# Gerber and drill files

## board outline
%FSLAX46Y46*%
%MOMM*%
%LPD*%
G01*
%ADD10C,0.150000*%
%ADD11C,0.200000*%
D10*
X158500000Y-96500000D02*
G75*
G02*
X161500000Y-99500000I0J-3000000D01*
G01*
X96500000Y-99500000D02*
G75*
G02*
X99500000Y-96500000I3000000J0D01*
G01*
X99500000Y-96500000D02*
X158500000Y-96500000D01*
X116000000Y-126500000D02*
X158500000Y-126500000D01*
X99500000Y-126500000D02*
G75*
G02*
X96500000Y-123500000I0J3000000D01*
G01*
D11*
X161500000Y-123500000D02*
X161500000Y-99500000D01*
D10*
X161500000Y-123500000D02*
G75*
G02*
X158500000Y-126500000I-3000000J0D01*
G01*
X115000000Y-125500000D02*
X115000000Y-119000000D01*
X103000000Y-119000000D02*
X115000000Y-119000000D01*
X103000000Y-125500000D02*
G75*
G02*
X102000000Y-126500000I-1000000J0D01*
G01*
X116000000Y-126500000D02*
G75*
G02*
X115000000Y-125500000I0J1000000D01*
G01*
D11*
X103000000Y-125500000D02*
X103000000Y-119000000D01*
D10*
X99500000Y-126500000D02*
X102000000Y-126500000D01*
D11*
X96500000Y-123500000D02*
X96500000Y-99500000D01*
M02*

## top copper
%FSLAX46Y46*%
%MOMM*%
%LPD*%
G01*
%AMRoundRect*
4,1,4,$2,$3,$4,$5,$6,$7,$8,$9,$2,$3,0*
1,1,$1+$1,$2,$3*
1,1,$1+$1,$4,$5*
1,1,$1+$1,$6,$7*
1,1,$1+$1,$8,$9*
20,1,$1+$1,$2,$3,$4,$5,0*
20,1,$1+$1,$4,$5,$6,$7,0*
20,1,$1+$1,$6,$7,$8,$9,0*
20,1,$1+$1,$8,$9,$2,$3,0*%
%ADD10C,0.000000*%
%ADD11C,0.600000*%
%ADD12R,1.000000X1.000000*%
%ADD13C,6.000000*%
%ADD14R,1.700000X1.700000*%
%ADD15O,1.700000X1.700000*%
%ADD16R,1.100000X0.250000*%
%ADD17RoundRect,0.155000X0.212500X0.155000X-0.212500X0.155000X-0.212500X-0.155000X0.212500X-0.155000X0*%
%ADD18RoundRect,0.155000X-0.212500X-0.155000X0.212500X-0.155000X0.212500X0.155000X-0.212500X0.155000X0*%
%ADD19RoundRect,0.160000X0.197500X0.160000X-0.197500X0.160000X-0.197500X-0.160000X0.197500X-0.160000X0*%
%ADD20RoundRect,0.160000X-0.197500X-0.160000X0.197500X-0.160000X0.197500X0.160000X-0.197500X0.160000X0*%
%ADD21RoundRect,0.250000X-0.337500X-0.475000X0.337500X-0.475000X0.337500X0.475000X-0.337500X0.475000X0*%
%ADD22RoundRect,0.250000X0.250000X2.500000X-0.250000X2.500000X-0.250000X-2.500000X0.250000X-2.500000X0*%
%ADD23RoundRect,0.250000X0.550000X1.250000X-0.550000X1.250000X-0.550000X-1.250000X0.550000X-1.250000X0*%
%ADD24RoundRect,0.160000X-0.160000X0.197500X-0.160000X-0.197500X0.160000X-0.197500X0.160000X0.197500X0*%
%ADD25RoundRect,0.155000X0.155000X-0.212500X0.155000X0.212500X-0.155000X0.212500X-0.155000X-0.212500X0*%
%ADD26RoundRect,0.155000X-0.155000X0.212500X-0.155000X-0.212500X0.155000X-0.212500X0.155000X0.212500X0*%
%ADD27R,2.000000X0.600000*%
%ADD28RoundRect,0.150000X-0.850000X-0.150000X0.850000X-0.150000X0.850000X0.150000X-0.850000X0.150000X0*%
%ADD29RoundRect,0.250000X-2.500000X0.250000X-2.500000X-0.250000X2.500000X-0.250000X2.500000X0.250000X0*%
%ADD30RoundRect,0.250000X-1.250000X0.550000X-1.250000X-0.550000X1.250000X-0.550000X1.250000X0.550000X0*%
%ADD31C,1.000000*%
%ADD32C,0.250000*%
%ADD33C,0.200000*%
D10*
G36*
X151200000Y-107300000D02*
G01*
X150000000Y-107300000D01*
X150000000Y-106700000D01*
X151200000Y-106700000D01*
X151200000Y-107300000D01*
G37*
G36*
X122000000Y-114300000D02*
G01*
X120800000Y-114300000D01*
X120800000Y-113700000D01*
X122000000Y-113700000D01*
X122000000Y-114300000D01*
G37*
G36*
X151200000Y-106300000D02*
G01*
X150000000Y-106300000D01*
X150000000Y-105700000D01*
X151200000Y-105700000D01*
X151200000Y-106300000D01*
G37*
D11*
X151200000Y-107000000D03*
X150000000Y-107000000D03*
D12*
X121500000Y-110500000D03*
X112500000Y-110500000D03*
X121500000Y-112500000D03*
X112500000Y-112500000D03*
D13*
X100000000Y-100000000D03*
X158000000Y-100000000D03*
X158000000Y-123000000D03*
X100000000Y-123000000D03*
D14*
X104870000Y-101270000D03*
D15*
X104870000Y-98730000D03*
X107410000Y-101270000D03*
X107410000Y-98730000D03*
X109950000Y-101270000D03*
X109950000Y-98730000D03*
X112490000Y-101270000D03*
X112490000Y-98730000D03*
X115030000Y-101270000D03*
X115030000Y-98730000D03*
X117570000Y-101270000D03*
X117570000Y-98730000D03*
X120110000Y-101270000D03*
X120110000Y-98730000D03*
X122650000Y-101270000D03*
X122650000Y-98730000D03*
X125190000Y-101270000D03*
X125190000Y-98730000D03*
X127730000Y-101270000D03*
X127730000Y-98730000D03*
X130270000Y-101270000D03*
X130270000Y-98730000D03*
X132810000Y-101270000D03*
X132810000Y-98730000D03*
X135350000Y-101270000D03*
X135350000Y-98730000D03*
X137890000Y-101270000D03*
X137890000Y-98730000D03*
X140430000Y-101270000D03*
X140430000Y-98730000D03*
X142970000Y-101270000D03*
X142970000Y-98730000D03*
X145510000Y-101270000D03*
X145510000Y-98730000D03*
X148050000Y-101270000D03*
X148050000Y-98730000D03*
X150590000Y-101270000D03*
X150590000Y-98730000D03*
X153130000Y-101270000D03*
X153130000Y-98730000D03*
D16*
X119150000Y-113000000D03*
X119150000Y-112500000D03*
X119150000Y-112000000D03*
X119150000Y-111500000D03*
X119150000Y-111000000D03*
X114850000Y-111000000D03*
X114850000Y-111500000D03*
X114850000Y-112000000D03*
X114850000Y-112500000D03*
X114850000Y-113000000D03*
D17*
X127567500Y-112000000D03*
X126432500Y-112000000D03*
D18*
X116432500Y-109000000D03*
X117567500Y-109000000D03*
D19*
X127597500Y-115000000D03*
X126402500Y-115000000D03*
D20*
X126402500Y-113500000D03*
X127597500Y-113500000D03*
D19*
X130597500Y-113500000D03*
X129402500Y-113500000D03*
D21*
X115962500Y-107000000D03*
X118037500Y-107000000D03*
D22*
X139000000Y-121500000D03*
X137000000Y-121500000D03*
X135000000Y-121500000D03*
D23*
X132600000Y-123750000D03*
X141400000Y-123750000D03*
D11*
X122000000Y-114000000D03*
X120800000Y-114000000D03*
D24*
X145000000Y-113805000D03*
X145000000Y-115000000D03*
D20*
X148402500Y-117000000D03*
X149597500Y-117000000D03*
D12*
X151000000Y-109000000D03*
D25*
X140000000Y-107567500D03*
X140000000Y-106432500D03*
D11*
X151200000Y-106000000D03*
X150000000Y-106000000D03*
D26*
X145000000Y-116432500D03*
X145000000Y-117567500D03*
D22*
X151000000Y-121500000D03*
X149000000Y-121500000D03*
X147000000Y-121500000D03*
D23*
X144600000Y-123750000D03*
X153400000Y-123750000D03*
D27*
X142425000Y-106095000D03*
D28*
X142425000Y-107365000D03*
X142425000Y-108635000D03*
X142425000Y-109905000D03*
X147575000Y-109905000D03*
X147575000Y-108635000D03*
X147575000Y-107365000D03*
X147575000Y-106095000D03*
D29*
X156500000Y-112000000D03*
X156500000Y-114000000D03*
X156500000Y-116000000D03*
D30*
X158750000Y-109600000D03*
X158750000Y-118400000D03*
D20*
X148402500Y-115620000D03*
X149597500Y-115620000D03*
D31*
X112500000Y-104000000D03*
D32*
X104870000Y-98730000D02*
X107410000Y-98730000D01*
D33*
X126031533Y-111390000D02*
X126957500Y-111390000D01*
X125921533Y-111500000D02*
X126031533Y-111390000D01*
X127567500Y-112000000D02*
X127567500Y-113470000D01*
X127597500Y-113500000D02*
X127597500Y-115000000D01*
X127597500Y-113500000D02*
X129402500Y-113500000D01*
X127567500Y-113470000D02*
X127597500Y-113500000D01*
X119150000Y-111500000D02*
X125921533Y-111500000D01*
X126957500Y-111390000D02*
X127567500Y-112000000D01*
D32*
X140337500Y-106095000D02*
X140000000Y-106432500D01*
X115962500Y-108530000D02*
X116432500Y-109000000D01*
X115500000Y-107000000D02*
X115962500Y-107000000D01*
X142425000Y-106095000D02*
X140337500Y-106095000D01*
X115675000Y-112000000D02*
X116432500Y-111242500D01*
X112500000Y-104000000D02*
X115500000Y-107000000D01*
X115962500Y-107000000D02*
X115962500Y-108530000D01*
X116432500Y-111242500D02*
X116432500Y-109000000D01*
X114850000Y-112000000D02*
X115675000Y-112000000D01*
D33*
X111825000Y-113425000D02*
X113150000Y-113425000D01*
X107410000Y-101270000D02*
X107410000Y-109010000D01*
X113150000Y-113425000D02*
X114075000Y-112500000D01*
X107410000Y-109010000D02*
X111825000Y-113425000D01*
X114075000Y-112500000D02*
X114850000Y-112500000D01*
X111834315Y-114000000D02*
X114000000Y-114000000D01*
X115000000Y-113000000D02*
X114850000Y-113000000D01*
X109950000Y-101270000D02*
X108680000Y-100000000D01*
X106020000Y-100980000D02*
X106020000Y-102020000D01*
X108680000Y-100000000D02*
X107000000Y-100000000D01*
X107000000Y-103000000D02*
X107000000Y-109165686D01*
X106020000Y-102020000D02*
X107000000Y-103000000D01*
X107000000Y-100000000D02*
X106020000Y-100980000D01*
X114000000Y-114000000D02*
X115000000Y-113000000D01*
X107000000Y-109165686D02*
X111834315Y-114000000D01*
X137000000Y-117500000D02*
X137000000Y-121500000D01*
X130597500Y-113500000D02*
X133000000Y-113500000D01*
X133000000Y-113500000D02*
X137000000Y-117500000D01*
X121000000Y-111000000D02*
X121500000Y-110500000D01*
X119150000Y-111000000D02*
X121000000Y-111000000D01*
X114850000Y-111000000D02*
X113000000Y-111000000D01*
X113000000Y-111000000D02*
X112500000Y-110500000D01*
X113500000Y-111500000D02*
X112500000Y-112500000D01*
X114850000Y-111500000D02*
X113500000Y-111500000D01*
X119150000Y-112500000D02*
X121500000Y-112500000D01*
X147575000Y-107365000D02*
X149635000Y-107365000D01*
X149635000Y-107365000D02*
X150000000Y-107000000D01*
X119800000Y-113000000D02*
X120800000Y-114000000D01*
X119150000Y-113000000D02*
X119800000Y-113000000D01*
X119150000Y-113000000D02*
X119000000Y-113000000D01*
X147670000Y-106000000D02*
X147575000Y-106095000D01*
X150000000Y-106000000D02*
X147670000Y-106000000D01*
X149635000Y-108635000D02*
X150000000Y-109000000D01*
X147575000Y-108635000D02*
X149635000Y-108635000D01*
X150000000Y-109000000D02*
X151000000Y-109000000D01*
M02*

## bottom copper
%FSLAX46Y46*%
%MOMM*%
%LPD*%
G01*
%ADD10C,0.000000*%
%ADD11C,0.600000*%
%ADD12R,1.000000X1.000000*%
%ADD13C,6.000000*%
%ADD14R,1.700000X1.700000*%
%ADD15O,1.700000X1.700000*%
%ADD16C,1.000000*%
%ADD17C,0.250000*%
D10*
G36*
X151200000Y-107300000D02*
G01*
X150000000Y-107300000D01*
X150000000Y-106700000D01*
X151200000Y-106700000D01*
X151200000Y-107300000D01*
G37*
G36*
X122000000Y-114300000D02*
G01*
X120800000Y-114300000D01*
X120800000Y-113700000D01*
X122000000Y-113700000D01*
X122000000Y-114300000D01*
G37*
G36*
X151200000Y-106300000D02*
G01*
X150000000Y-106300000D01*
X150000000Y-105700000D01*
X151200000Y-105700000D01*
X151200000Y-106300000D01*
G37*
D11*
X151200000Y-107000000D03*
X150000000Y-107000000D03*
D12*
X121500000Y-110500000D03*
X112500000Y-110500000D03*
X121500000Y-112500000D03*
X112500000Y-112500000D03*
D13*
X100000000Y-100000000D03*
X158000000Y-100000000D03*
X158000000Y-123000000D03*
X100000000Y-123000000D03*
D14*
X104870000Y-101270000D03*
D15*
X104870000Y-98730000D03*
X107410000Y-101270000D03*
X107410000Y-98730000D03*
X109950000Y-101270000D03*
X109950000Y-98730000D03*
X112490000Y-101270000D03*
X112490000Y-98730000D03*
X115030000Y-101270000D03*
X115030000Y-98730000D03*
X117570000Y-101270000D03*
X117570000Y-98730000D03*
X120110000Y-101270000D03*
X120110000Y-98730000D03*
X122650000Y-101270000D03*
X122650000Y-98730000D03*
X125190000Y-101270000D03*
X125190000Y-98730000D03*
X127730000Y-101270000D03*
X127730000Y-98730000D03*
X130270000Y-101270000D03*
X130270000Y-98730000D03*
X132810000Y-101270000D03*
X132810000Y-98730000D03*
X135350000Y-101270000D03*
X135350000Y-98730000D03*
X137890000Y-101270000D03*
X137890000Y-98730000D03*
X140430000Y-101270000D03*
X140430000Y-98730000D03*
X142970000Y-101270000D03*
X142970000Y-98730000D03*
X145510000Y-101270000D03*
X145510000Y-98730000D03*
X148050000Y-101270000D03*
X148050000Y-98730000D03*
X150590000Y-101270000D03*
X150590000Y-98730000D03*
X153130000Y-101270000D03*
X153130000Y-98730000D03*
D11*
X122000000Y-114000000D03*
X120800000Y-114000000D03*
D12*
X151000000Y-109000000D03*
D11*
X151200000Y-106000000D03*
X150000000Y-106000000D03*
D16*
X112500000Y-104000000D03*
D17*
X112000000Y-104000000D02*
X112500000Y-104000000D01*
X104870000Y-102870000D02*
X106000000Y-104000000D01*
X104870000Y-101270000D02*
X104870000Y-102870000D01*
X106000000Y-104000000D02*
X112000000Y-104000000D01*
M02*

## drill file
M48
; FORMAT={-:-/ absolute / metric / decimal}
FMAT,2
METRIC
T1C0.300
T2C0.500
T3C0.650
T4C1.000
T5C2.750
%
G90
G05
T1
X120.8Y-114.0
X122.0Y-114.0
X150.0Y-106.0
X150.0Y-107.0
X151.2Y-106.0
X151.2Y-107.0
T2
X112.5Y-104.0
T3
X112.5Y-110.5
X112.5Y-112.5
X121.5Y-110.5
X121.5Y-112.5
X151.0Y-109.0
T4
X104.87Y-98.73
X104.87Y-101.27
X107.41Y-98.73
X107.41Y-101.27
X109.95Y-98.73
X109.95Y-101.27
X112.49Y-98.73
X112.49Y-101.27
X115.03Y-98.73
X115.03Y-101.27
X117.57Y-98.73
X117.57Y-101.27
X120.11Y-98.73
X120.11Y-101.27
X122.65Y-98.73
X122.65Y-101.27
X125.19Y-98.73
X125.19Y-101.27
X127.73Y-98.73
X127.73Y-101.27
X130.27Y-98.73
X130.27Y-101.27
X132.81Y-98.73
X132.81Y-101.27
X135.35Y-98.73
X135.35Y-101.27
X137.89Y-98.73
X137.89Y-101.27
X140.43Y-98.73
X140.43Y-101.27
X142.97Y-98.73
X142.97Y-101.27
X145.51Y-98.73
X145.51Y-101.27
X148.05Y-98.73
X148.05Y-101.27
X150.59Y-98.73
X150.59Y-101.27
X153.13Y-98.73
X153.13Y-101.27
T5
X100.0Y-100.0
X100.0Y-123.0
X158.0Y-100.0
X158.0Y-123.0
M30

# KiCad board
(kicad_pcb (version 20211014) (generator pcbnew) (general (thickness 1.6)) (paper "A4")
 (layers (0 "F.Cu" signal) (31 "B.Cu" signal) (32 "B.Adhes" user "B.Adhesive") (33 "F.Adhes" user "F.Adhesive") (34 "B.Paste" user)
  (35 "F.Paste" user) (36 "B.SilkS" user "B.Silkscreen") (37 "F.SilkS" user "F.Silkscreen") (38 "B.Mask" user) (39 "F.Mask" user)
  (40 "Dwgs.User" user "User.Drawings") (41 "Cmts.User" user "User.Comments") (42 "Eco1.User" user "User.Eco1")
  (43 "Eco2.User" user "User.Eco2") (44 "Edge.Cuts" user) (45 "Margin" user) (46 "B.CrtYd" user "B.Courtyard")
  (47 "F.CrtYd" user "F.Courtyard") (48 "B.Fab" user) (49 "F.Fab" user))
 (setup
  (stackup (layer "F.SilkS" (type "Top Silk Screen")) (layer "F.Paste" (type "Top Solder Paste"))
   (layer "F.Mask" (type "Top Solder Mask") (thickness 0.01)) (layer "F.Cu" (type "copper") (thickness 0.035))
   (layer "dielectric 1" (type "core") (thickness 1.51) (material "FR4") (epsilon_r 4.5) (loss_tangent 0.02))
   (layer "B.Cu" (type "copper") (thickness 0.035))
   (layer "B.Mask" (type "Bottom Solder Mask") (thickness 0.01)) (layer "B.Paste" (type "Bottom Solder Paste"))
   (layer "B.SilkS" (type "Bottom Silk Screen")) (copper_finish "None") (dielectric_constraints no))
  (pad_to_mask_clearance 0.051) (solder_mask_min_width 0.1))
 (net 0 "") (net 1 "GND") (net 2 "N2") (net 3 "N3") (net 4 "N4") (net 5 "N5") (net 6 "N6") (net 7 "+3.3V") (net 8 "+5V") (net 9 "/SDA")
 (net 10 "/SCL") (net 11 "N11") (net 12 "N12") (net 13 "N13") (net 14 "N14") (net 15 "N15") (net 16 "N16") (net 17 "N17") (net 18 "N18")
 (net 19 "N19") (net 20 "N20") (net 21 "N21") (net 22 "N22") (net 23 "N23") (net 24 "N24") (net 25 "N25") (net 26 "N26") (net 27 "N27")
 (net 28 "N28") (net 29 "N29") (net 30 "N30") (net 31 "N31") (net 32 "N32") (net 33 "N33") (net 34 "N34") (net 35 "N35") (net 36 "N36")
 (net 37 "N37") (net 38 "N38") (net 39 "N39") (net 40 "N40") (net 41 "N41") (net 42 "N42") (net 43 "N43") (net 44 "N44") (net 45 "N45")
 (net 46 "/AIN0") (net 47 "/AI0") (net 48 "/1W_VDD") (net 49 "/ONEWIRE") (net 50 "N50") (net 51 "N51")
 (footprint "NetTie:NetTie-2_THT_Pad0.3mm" (layer "F.Cu") (at 151.2 107 180)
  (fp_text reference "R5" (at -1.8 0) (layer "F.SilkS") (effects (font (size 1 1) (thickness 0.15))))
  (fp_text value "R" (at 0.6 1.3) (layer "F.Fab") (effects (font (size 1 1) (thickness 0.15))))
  (fp_poly (pts (xy 0 -0.3) (xy 1.2 -0.3) (xy 1.2 0.3) (xy 0 0.3)) (layer "F.Cu") (width 0) (fill solid))
  (fp_poly (pts (xy 0 -0.3) (xy 1.2 -0.3) (xy 1.2 0.3) (xy 0 0.3)) (layer "B.Cu") (width 0) (fill solid))
  (pad "1" thru_hole circle (at 0 0 180) (size 0.6 0.6) (drill 0.3) (layers *.Cu) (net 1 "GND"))
  (pad "2" thru_hole circle (at 1.2 0 180) (size 0.6 0.6) (drill 0.3) (layers *.Cu) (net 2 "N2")))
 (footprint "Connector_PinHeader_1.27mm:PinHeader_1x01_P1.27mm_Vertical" (layer "F.Cu") (at 121.5 110.5 -90)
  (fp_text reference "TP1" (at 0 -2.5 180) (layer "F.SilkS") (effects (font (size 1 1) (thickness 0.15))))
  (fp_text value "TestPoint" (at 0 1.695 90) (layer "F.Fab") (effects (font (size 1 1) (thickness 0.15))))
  (pad "1" thru_hole rect (at 0 0 270) (size 1 1) (drill 0.65) (layers *.Cu *.Mask) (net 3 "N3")))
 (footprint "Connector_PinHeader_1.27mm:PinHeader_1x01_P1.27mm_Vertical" (layer "F.Cu") (at 112.5 110.5 90)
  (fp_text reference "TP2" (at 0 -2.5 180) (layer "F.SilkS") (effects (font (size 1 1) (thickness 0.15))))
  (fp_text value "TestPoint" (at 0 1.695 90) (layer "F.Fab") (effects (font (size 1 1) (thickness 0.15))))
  (pad "1" thru_hole rect (at 0 0 90) (size 1 1) (drill 0.65) (layers *.Cu *.Mask) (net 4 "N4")))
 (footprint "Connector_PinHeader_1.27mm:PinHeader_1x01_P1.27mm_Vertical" (layer "F.Cu") (at 121.5 112.5 -90)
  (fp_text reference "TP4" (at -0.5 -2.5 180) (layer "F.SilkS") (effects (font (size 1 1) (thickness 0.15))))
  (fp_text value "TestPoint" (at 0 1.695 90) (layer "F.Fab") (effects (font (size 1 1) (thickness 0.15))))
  (pad "1" thru_hole rect (at 0 0 270) (size 1 1) (drill 0.65) (layers *.Cu *.Mask) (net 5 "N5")))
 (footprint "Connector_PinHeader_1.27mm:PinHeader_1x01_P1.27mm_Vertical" (layer "F.Cu") (at 112.5 112.5 90)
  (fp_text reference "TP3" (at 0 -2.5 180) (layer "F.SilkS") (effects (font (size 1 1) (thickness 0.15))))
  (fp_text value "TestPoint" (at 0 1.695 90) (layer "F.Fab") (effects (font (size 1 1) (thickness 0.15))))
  (pad "1" thru_hole rect (at 0 0 90) (size 1 1) (drill 0.65) (layers *.Cu *.Mask) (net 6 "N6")))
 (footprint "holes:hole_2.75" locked (layer "F.Cu") (at 100 100)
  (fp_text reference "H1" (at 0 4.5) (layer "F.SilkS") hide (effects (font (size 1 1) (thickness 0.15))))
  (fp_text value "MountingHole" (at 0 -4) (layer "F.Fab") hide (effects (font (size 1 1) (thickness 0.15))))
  (pad "" np_thru_hole circle locked (at 0 0) (size 6 6) (drill 2.75) (layers *.Cu *.Mask)))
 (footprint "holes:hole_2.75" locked (layer "F.Cu") (at 158 100)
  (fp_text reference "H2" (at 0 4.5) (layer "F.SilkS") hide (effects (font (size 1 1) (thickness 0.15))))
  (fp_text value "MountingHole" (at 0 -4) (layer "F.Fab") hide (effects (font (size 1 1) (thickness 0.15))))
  (pad "" np_thru_hole circle locked (at 0 0) (size 6 6) (drill 2.75) (layers *.Cu *.Mask)))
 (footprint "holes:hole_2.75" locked (layer "F.Cu") (at 158 123)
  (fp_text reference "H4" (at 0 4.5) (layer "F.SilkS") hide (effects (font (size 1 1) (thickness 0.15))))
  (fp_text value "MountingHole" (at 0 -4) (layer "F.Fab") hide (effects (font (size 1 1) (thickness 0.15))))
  (pad "" np_thru_hole circle locked (at 0 0) (size 6 6) (drill 2.75) (layers *.Cu *.Mask)))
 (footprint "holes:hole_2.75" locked (layer "F.Cu") (at 100 123)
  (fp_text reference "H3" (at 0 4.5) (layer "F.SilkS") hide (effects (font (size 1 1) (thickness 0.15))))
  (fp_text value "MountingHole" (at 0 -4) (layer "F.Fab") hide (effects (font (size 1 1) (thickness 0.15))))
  (pad "" np_thru_hole circle locked (at 0 0) (size 6 6) (drill 2.75) (layers *.Cu *.Mask)))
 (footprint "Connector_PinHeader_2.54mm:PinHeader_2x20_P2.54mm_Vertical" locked (layer "F.Cu") (at 104.87 101.27 90)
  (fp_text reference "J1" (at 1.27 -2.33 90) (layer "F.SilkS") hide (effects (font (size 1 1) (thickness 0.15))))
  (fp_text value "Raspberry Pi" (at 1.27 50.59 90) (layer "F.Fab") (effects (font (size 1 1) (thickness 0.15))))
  (pad "1" thru_hole rect locked (at 0 0 90) (size 1.7 1.7) (drill 1) (layers *.Cu *.Mask) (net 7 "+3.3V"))
  (pad "2" thru_hole oval locked (at 2.54 0 90) (size 1.7 1.7) (drill 1) (layers *.Cu *.Mask) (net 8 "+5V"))
  (pad "3" thru_hole oval locked (at 0 2.54 90) (size 1.7 1.7) (drill 1) (layers *.Cu *.Mask) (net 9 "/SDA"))
  (pad "4" thru_hole oval locked (at 2.54 2.54 90) (size 1.7 1.7) (drill 1) (layers *.Cu *.Mask) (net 8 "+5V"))
  (pad "5" thru_hole oval locked (at 0 5.08 90) (size 1.7 1.7) (drill 1) (layers *.Cu *.Mask) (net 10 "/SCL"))
  (pad "6" thru_hole oval locked (at 2.54 5.08 90) (size 1.7 1.7) (drill 1) (layers *.Cu *.Mask) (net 1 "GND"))
  (pad "7" thru_hole oval locked (at 0 7.62 90) (size 1.7 1.7) (drill 1) (layers *.Cu *.Mask) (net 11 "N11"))
  (pad "8" thru_hole oval locked (at 2.54 7.62 90) (size 1.7 1.7) (drill 1) (layers *.Cu *.Mask) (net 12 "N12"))
  (pad "9" thru_hole oval locked (at 0 10.16 90) (size 1.7 1.7) (drill 1) (layers *.Cu *.Mask) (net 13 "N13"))
  (pad "10" thru_hole oval locked (at 2.54 10.16 90) (size 1.7 1.7) (drill 1) (layers *.Cu *.Mask) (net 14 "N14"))
  (pad "11" thru_hole oval locked (at 0 12.7 90) (size 1.7 1.7) (drill 1) (layers *.Cu *.Mask) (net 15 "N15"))
  (pad "12" thru_hole oval locked (at 2.54 12.7 90) (size 1.7 1.7) (drill 1) (layers *.Cu *.Mask) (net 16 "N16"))
  (pad "13" thru_hole oval locked (at 0 15.24 90) (size 1.7 1.7) (drill 1) (layers *.Cu *.Mask) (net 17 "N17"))
  (pad "14" thru_hole oval locked (at 2.54 15.24 90) (size 1.7 1.7) (drill 1) (layers *.Cu *.Mask) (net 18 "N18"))
  (pad "15" thru_hole oval locked (at 0 17.78 90) (size 1.7 1.7) (drill 1) (layers *.Cu *.Mask) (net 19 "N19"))
  (pad "16" thru_hole oval locked (at 2.54 17.78 90) (size 1.7 1.7) (drill 1) (layers *.Cu *.Mask) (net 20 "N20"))
  (pad "17" thru_hole oval locked (at 0 20.32 90) (size 1.7 1.7) (drill 1) (layers *.Cu *.Mask) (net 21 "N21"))
  (pad "18" thru_hole oval locked (at 2.54 20.32 90) (size 1.7 1.7) (drill 1) (layers *.Cu *.Mask) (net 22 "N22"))
  (pad "19" thru_hole oval locked (at 0 22.86 90) (size 1.7 1.7) (drill 1) (layers *.Cu *.Mask) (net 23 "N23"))
  (pad "20" thru_hole oval locked (at 2.54 22.86 90) (size 1.7 1.7) (drill 1) (layers *.Cu *.Mask) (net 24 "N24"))
  (pad "21" thru_hole oval locked (at 0 25.4 90) (size 1.7 1.7) (drill 1) (layers *.Cu *.Mask) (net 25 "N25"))
  (pad "22" thru_hole oval locked (at 2.54 25.4 90) (size 1.7 1.7) (drill 1) (layers *.Cu *.Mask) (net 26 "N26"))
  (pad "23" thru_hole oval locked (at 0 27.94 90) (size 1.7 1.7) (drill 1) (layers *.Cu *.Mask) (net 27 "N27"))
  (pad "24" thru_hole oval locked (at 2.54 27.94 90) (size 1.7 1.7) (drill 1) (layers *.Cu *.Mask) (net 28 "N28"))
  (pad "25" thru_hole oval locked (at 0 30.48 90) (size 1.7 1.7) (drill 1) (layers *.Cu *.Mask) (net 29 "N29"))
  (pad "26" thru_hole oval locked (at 2.54 30.48 90) (size 1.7 1.7) (drill 1) (layers *.Cu *.Mask) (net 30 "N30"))
  (pad "27" thru_hole oval locked (at 0 33.02 90) (size 1.7 1.7) (drill 1) (layers *.Cu *.Mask) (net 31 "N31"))
  (pad "28" thru_hole oval locked (at 2.54 33.02 90) (size 1.7 1.7) (drill 1) (layers *.Cu *.Mask) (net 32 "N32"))
  (pad "29" thru_hole oval locked (at 0 35.56 90) (size 1.7 1.7) (drill 1) (layers *.Cu *.Mask) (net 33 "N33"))
  (pad "30" thru_hole oval locked (at 2.54 35.56 90) (size 1.7 1.7) (drill 1) (layers *.Cu *.Mask) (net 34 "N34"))
  (pad "31" thru_hole oval locked (at 0 38.1 90) (size 1.7 1.7) (drill 1) (layers *.Cu *.Mask) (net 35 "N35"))
  (pad "32" thru_hole oval locked (at 2.54 38.1 90) (size 1.7 1.7) (drill 1) (layers *.Cu *.Mask) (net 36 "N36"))
  (pad "33" thru_hole oval locked (at 0 40.64 90) (size 1.7 1.7) (drill 1) (layers *.Cu *.Mask) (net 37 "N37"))
  (pad "34" thru_hole oval locked (at 2.54 40.64 90) (size 1.7 1.7) (drill 1) (layers *.Cu *.Mask) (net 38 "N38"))
  (pad "35" thru_hole oval locked (at 0 43.18 90) (size 1.7 1.7) (drill 1) (layers *.Cu *.Mask) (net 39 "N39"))
  (pad "36" thru_hole oval locked (at 2.54 43.18 90) (size 1.7 1.7) (drill 1) (layers *.Cu *.Mask) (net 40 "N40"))
  (pad "37" thru_hole oval locked (at 0 45.72 90) (size 1.7 1.7) (drill 1) (layers *.Cu *.Mask) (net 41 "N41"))
  (pad "38" thru_hole oval locked (at 2.54 45.72 90) (size 1.7 1.7) (drill 1) (layers *.Cu *.Mask) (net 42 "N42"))
  (pad "39" thru_hole oval locked (at 0 48.26 90) (size 1.7 1.7) (drill 1) (layers *.Cu *.Mask) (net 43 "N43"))
  (pad "40" thru_hole oval locked (at 2.54 48.26 90) (size 1.7 1.7) (drill 1) (layers *.Cu *.Mask) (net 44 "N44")))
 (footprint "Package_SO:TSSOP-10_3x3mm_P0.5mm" (layer "F.Cu") (at 117 112 180)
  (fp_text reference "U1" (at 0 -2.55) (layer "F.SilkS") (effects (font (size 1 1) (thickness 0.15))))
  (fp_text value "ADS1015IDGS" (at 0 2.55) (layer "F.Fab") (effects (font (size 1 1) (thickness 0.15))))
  (pad "1" smd rect (at -2.15 -1 180) (size 1.1 0.25) (layers "F.Cu" "F.Paste" "F.Mask") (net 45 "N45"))
  (pad "2" smd rect (at -2.15 -0.5 180) (size 1.1 0.25) (layers "F.Cu" "F.Paste" "F.Mask") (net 5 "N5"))
  (pad "3" smd rect (at -2.15 0 180) (size 1.1 0.25) (layers "F.Cu" "F.Paste" "F.Mask") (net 1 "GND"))
  (pad "4" smd rect (at -2.15 0.5 180) (size 1.1 0.25) (layers "F.Cu" "F.Paste" "F.Mask") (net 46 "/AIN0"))
  (pad "5" smd rect (at -2.15 1 180) (size 1.1 0.25) (layers "F.Cu" "F.Paste" "F.Mask") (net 3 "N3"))
  (pad "6" smd rect (at 2.15 1 180) (size 1.1 0.25) (layers "F.Cu" "F.Paste" "F.Mask") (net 4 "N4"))
  (pad "7" smd rect (at 2.15 0.5 180) (size 1.1 0.25) (layers "F.Cu" "F.Paste" "F.Mask") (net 6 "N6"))
  (pad "8" smd rect (at 2.15 0 180) (size 1.1 0.25) (layers "F.Cu" "F.Paste" "F.Mask") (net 7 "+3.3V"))
  (pad "9" smd rect (at 2.15 -0.5 180) (size 1.1 0.25) (layers "F.Cu" "F.Paste" "F.Mask") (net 9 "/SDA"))
  (pad "10" smd rect (at 2.15 -1 180) (size 1.1 0.25) (layers "F.Cu" "F.Paste" "F.Mask") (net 10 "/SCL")))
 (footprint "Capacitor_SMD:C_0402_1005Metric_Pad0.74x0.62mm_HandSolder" (layer "F.Cu") (at 127 112 180)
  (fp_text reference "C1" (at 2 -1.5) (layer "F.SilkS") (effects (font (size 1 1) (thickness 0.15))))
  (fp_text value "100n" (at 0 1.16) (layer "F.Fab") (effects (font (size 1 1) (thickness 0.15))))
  (pad "1" smd roundrect (at -0.5675 0 180) (size 0.735 0.62) (layers "F.Cu" "F.Paste" "F.Mask") (roundrect_rratio 0.25) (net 46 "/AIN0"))
  (pad "2" smd roundrect (at 0.5675 0 180) (size 0.735 0.62) (layers "F.Cu" "F.Paste" "F.Mask") (roundrect_rratio 0.25) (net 1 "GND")))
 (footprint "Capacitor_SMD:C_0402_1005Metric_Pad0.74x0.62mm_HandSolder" (layer "F.Cu") (at 117 109)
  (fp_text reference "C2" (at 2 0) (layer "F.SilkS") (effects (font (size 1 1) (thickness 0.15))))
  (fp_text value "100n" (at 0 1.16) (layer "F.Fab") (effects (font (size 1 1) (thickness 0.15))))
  (pad "1" smd roundrect (at -0.5675 0) (size 0.735 0.62) (layers "F.Cu" "F.Paste" "F.Mask") (roundrect_rratio 0.25) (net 7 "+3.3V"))
  (pad "2" smd roundrect (at 0.5675 0) (size 0.735 0.62) (layers "F.Cu" "F.Paste" "F.Mask") (roundrect_rratio 0.25) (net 1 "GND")))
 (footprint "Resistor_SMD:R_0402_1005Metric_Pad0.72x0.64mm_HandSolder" (layer "F.Cu") (at 127 115 180)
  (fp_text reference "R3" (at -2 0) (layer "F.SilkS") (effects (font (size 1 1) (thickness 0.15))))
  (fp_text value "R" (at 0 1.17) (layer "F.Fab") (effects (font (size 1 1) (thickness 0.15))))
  (pad "1" smd roundrect (at -0.5975 0 180) (size 0.715 0.64) (layers "F.Cu" "F.Paste" "F.Mask") (roundrect_rratio 0.25) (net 46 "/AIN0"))
  (pad "2" smd roundrect (at 0.5975 0 180) (size 0.715 0.64) (layers "F.Cu" "F.Paste" "F.Mask") (roundrect_rratio 0.25) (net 7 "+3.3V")))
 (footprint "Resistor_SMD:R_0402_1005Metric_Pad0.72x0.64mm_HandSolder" (layer "F.Cu") (at 127 113.5)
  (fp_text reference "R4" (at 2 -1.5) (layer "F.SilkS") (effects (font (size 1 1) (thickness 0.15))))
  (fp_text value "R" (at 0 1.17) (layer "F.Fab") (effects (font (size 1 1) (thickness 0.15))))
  (pad "1" smd roundrect (at -0.5975 0) (size 0.715 0.64) (layers "F.Cu" "F.Paste" "F.Mask") (roundrect_rratio 0.25) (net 1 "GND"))
  (pad "2" smd roundrect (at 0.5975 0) (size 0.715 0.64) (layers "F.Cu" "F.Paste" "F.Mask") (roundrect_rratio 0.25) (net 46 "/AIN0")))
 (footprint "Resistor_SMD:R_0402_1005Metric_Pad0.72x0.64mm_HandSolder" (layer "F.Cu") (at 130 113.5 180)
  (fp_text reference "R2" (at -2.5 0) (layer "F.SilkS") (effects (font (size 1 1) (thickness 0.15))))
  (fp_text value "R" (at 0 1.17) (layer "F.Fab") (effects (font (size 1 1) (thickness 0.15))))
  (pad "1" smd roundrect (at -0.5975 0 180) (size 0.715 0.64) (layers "F.Cu" "F.Paste" "F.Mask") (roundrect_rratio 0.25) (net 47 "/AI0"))
  (pad "2" smd roundrect (at 0.5975 0 180) (size 0.715 0.64) (layers "F.Cu" "F.Paste" "F.Mask") (roundrect_rratio 0.25) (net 46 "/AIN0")))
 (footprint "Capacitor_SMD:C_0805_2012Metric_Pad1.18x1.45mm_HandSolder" (layer "F.Cu") (at 117 107)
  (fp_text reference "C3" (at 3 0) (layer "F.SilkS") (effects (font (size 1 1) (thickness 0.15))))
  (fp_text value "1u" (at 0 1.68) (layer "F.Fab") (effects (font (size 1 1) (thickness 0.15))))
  (pad "1" smd roundrect (at -1.0375 0) (size 1.175 1.45) (layers "F.Cu" "F.Paste" "F.Mask") (roundrect_rratio 0.212766) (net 7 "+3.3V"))
  (pad "2" smd roundrect (at 1.0375 0) (size 1.175 1.45) (layers "F.Cu" "F.Paste" "F.Mask") (roundrect_rratio 0.212766) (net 1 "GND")))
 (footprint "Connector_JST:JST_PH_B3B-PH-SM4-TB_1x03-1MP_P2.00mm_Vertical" (layer "F.Cu") (at 137 122 180)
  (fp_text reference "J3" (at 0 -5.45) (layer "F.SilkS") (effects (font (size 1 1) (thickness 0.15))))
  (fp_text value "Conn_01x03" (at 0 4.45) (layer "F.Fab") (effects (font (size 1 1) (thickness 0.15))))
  (pad "1" smd roundrect (at -2 0.5 180) (size 1 5.5) (layers "F.Cu" "F.Paste" "F.Mask") (roundrect_rratio 0.25) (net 1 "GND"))
  (pad "2" smd roundrect (at 0 0.5 180) (size 1 5.5) (layers "F.Cu" "F.Paste" "F.Mask") (roundrect_rratio 0.25) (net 47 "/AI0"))
  (pad "3" smd roundrect (at 2 0.5 180) (size 1 5.5) (layers "F.Cu" "F.Paste" "F.Mask") (roundrect_rratio 0.25) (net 7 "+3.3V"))
  (pad "MP" smd roundrect (at 4.4 -1.75 180) (size 1.6 3) (layers "F.Cu" "F.Paste" "F.Mask") (roundrect_rratio 0.15625))
  (pad "MP" smd roundrect (at -4.4 -1.75 180) (size 1.6 3) (layers "F.Cu" "F.Paste" "F.Mask") (roundrect_rratio 0.15625)))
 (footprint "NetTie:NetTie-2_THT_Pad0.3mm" (layer "F.Cu") (at 122 114 180)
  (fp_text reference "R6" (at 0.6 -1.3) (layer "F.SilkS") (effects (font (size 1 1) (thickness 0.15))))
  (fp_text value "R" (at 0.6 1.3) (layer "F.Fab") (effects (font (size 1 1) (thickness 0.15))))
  (fp_poly (pts (xy 0 -0.3) (xy 1.2 -0.3) (xy 1.2 0.3) (xy 0 0.3)) (layer "F.Cu") (width 0) (fill solid))
  (fp_poly (pts (xy 0 -0.3) (xy 1.2 -0.3) (xy 1.2 0.3) (xy 0 0.3)) (layer "B.Cu") (width 0) (fill solid))
  (pad "1" thru_hole circle (at 0 0 180) (size 0.6 0.6) (drill 0.3) (layers *.Cu) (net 1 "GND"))
  (pad "2" thru_hole circle (at 1.2 0 180) (size 0.6 0.6) (drill 0.3) (layers *.Cu) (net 45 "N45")))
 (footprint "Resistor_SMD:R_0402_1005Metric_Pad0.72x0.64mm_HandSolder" (layer "F.Cu") (at 145 114.4025 -90)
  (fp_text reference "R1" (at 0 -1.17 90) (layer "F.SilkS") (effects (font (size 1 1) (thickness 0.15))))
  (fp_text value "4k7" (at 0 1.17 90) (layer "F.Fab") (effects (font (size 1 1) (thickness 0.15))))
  (pad "1" smd roundrect (at -0.5975 0 270) (size 0.715 0.64) (layers "F.Cu" "F.Paste" "F.Mask") (roundrect_rratio 0.25) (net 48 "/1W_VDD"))
  (pad "2" smd roundrect (at 0.5975 0 270) (size 0.715 0.64) (layers "F.Cu" "F.Paste" "F.Mask") (roundrect_rratio 0.25) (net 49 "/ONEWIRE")))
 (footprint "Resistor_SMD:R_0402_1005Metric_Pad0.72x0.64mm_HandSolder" (layer "F.Cu") (at 149 117)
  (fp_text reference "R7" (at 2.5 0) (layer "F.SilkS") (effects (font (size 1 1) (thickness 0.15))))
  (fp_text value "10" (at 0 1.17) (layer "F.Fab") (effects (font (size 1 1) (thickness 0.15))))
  (pad "1" smd roundrect (at -0.5975 0) (size 0.715 0.64) (layers "F.Cu" "F.Paste" "F.Mask") (roundrect_rratio 0.25) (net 11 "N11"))
  (pad "2" smd roundrect (at 0.5975 0) (size 0.715 0.64) (layers "F.Cu" "F.Paste" "F.Mask") (roundrect_rratio 0.25) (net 49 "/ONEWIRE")))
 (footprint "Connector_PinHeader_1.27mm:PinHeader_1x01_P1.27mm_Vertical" (layer "F.Cu") (at 151 109)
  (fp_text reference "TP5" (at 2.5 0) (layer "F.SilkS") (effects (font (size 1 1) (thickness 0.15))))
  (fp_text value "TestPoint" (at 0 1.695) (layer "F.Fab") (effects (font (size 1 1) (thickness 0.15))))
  (pad "1" thru_hole rect (at 0 0) (size 1 1) (drill 0.65) (layers *.Cu *.Mask) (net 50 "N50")))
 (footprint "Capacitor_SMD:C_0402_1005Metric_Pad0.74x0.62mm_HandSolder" (layer "F.Cu") (at 140 107 90)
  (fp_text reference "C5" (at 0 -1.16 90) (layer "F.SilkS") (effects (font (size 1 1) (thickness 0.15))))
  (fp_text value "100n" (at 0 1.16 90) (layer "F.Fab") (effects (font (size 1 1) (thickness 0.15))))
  (pad "1" smd roundrect (at -0.5675 0 90) (size 0.735 0.62) (layers "F.Cu" "F.Paste" "F.Mask") (roundrect_rratio 0.25) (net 1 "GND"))
  (pad "2" smd roundrect (at 0.5675 0 90) (size 0.735 0.62) (layers "F.Cu" "F.Paste" "F.Mask") (roundrect_rratio 0.25) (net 7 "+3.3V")))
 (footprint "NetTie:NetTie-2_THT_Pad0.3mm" (layer "F.Cu") (at 151.2 106 180)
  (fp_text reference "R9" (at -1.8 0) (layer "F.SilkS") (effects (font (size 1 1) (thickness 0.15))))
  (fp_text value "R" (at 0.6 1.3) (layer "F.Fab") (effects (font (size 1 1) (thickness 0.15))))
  (fp_poly (pts (xy 0 -0.3) (xy 1.2 -0.3) (xy 1.2 0.3) (xy 0 0.3)) (layer "F.Cu") (width 0) (fill solid))
  (fp_poly (pts (xy 0 -0.3) (xy 1.2 -0.3) (xy 1.2 0.3) (xy 0 0.3)) (layer "B.Cu") (width 0) (fill solid))
  (pad "1" thru_hole circle (at 0 0 180) (size 0.6 0.6) (drill 0.3) (layers *.Cu) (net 1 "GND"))
  (pad "2" thru_hole circle (at 1.2 0 180) (size 0.6 0.6) (drill 0.3) (layers *.Cu) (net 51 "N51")))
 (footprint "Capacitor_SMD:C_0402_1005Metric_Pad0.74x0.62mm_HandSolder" (layer "F.Cu") (at 145 117 -90)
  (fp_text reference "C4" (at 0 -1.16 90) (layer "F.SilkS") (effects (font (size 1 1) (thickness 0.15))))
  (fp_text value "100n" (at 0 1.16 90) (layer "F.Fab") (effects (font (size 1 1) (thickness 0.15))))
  (pad "1" smd roundrect (at -0.5675 0 270) (size 0.735 0.62) (layers "F.Cu" "F.Paste" "F.Mask") (roundrect_rratio 0.25) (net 1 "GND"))
  (pad "2" smd roundrect (at 0.5675 0 270) (size 0.735 0.62) (layers "F.Cu" "F.Paste" "F.Mask") (roundrect_rratio 0.25) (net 48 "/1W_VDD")))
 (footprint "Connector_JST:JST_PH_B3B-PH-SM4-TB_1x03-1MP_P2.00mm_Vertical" (layer "F.Cu") (at 149 122 180)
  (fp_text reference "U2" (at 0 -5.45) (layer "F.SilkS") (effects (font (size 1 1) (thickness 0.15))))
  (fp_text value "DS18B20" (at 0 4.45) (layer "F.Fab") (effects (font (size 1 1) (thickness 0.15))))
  (pad "1" smd roundrect (at -2 0.5 180) (size 1 5.5) (layers "F.Cu" "F.Paste" "F.Mask") (roundrect_rratio 0.25) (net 1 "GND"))
  (pad "2" smd roundrect (at 0 0.5 180) (size 1 5.5) (layers "F.Cu" "F.Paste" "F.Mask") (roundrect_rratio 0.25) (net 49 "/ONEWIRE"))
  (pad "3" smd roundrect (at 2 0.5 180) (size 1 5.5) (layers "F.Cu" "F.Paste" "F.Mask") (roundrect_rratio 0.25) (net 48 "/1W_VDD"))
  (pad "MP" smd roundrect (at 4.4 -1.75 180) (size 1.6 3) (layers "F.Cu" "F.Paste" "F.Mask") (roundrect_rratio 0.15625))
  (pad "MP" smd roundrect (at -4.4 -1.75 180) (size 1.6 3) (layers "F.Cu" "F.Paste" "F.Mask") (roundrect_rratio 0.15625)))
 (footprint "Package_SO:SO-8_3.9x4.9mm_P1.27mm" (layer "F.Cu") (at 145 108)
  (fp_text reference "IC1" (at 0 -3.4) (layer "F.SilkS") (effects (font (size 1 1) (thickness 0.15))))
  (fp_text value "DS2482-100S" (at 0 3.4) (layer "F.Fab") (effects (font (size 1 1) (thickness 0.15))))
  (pad "1" smd rect (at -2.575 -1.905) (size 2 0.6) (layers "F.Cu" "F.Paste" "F.Mask") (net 7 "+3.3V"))
  (pad "2" smd roundrect (at -2.575 -0.635) (size 2 0.6) (layers "F.Cu" "F.Paste" "F.Mask") (roundrect_rratio 0.25) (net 49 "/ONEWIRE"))
  (pad "3" smd roundrect (at -2.575 0.635) (size 2 0.6) (layers "F.Cu" "F.Paste" "F.Mask") (roundrect_rratio 0.25) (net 1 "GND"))
  (pad "4" smd roundrect (at -2.575 1.905) (size 2 0.6) (layers "F.Cu" "F.Paste" "F.Mask") (roundrect_rratio 0.25) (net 10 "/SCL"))
  (pad "5" smd roundrect (at 2.575 1.905) (size 2 0.6) (layers "F.Cu" "F.Paste" "F.Mask") (roundrect_rratio 0.25) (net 9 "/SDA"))
  (pad "6" smd roundrect (at 2.575 0.635) (size 2 0.6) (layers "F.Cu" "F.Paste" "F.Mask") (roundrect_rratio 0.25) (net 50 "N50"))
  (pad "7" smd roundrect (at 2.575 -0.635) (size 2 0.6) (layers "F.Cu" "F.Paste" "F.Mask") (roundrect_rratio 0.25) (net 2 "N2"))
  (pad "8" smd roundrect (at 2.575 -1.905) (size 2 0.6) (layers "F.Cu" "F.Paste" "F.Mask") (roundrect_rratio 0.25) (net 51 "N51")))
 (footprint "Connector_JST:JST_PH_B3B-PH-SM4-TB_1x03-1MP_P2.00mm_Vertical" (layer "F.Cu") (at 157 114 -90)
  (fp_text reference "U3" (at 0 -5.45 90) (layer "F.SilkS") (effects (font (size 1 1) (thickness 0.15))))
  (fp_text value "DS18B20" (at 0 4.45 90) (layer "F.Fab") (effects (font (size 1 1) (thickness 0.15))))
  (pad "1" smd roundrect (at -2 0.5 270) (size 1 5.5) (layers "F.Cu" "F.Paste" "F.Mask") (roundrect_rratio 0.25) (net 1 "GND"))
  (pad "2" smd roundrect (at 0 0.5 270) (size 1 5.5) (layers "F.Cu" "F.Paste" "F.Mask") (roundrect_rratio 0.25) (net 49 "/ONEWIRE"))
  (pad "3" smd roundrect (at 2 0.5 270) (size 1 5.5) (layers "F.Cu" "F.Paste" "F.Mask") (roundrect_rratio 0.25) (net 48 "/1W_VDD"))
  (pad "MP" smd roundrect (at -4.4 -1.75 270) (size 1.6 3) (layers "F.Cu" "F.Paste" "F.Mask") (roundrect_rratio 0.15625))
  (pad "MP" smd roundrect (at 4.4 -1.75 270) (size 1.6 3) (layers "F.Cu" "F.Paste" "F.Mask") (roundrect_rratio 0.15625)))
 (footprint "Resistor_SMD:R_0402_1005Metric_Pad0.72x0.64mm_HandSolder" (layer "F.Cu") (at 149 115.62)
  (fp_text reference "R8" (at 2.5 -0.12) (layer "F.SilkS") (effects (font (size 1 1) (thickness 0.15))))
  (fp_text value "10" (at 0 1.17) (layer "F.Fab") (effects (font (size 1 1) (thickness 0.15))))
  (pad "1" smd roundrect (at -0.5975 0) (size 0.715 0.64) (layers "F.Cu" "F.Paste" "F.Mask") (roundrect_rratio 0.25) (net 7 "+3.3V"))
  (pad "2" smd roundrect (at 0.5975 0) (size 0.715 0.64) (layers "F.Cu" "F.Paste" "F.Mask") (roundrect_rratio 0.25) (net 48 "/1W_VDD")))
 (gr_arc (start 158.5 96.5) (mid 160.62132 97.37868) (end 161.5 99.5) (layer "Edge.Cuts") (width 0.15))
 (gr_arc (start 96.5 99.5) (mid 97.37868 97.37868) (end 99.5 96.5) (layer "Edge.Cuts") (width 0.15))
 (gr_line (start 99.5 96.5) (end 158.5 96.5) (layer "Edge.Cuts") (width 0.15))
 (gr_line (start 116 126.5) (end 158.5 126.5) (layer "Edge.Cuts") (width 0.15))
 (gr_arc (start 99.5 126.5) (mid 97.37868 125.62132) (end 96.5 123.5) (layer "Edge.Cuts") (width 0.15))
 (gr_line (start 161.5 123.5) (end 161.5 99.5) (layer "Edge.Cuts") (width 0.2))
 (gr_arc (start 161.5 123.5) (mid 160.62132 125.62132) (end 158.5 126.5) (layer "Edge.Cuts") (width 0.15))
 (gr_line (start 115 125.5) (end 115 119) (layer "Edge.Cuts") (width 0.15))
 (gr_line (start 103 119) (end 115 119) (layer "Edge.Cuts") (width 0.15))
 (gr_arc (start 103 125.5) (mid 102.707107 126.207107) (end 102 126.5) (layer "Edge.Cuts") (width 0.15))
 (gr_arc (start 116 126.5) (mid 115.292893 126.207107) (end 115 125.5) (layer "Edge.Cuts") (width 0.15))
 (gr_line (start 103 125.5) (end 103 119) (layer "Edge.Cuts") (width 0.2))
 (gr_line (start 99.5 126.5) (end 102 126.5) (layer "Edge.Cuts") (width 0.15))
 (gr_line (start 96.5 123.5) (end 96.5 99.5) (layer "Edge.Cuts") (width 0.2))
 (segment (start 104.87 98.73) (end 107.41 98.73) (width 0.25) (layer "F.Cu") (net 8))
 (segment (start 126.031533 111.39) (end 126.9575 111.39) (width 0.2) (layer "F.Cu") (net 46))
 (segment (start 125.921533 111.5) (end 126.031533 111.39) (width 0.2) (layer "F.Cu") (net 46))
 (segment (start 127.5675 112) (end 127.5675 113.47) (width 0.2) (layer "F.Cu") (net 46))
 (segment (start 127.5975 113.5) (end 127.5975 115) (width 0.2) (layer "F.Cu") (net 46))
 (segment (start 127.5975 113.5) (end 129.4025 113.5) (width 0.2) (layer "F.Cu") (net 46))
 (segment (start 127.5675 113.47) (end 127.5975 113.5) (width 0.2) (layer "F.Cu") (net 46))
 (segment (start 119.15 111.5) (end 125.921533 111.5) (width 0.2) (layer "F.Cu") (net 46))
 (segment (start 126.9575 111.39) (end 127.5675 112) (width 0.2) (layer "F.Cu") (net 46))
 (segment (start 140.3375 106.095) (end 140 106.4325) (width 0.25) (layer "F.Cu") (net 7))
 (segment (start 115.9625 108.53) (end 116.4325 109) (width 0.25) (layer "F.Cu") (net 7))
 (segment (start 115.5 107) (end 115.9625 107) (width 0.25) (layer "F.Cu") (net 7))
 (segment (start 142.425 106.095) (end 140.3375 106.095) (width 0.25) (layer "F.Cu") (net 7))
 (segment (start 115.675 112) (end 116.4325 111.2425) (width 0.25) (layer "F.Cu") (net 7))
 (segment (start 112.5 104) (end 115.5 107) (width 0.25) (layer "F.Cu") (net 7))
 (segment (start 115.9625 107) (end 115.9625 108.53) (width 0.25) (layer "F.Cu") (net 7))
 (segment (start 116.4325 111.2425) (end 116.4325 109) (width 0.25) (layer "F.Cu") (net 7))
 (segment (start 114.85 112) (end 115.675 112) (width 0.25) (layer "F.Cu") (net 7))
 (via (at 112.5 104) (size 1) (drill 0.5) (layers "F.Cu" "B.Cu") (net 7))
 (segment (start 112 104) (end 112.5 104) (width 0.25) (layer "B.Cu") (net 7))
 (segment (start 104.87 102.87) (end 106 104) (width 0.25) (layer "B.Cu") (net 7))
 (segment (start 104.87 101.27) (end 104.87 102.87) (width 0.25) (layer "B.Cu") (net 7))
 (segment (start 106 104) (end 112 104) (width 0.25) (layer "B.Cu") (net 7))
 (segment (start 111.825 113.425) (end 113.15 113.425) (width 0.2) (layer "F.Cu") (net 9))
 (segment (start 107.41 101.27) (end 107.41 109.01) (width 0.2) (layer "F.Cu") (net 9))
 (segment (start 113.15 113.425) (end 114.075 112.5) (width 0.2) (layer "F.Cu") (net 9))
 (segment (start 107.41 109.01) (end 111.825 113.425) (width 0.2) (layer "F.Cu") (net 9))
 (segment (start 114.075 112.5) (end 114.85 112.5) (width 0.2) (layer "F.Cu") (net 9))
 (segment (start 111.834315 114) (end 114 114) (width 0.2) (layer "F.Cu") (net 10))
 (segment (start 115 113) (end 114.85 113) (width 0.2) (layer "F.Cu") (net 10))
 (segment (start 109.95 101.27) (end 108.68 100) (width 0.2) (layer "F.Cu") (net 10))
 (segment (start 106.02 100.98) (end 106.02 102.02) (width 0.2) (layer "F.Cu") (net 10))
 (segment (start 108.68 100) (end 107 100) (width 0.2) (layer "F.Cu") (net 10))
 (segment (start 107 103) (end 107 109.165686) (width 0.2) (layer "F.Cu") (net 10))
 (segment (start 106.02 102.02) (end 107 103) (width 0.2) (layer "F.Cu") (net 10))
 (segment (start 107 100) (end 106.02 100.98) (width 0.2) (layer "F.Cu") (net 10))
 (segment (start 114 114) (end 115 113) (width 0.2) (layer "F.Cu") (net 10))
 (segment (start 107 109.165686) (end 111.834315 114) (width 0.2) (layer "F.Cu") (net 10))
 (segment (start 137 117.5) (end 137 121.5) (width 0.2) (layer "F.Cu") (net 47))
 (segment (start 130.5975 113.5) (end 133 113.5) (width 0.2) (layer "F.Cu") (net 47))
 (segment (start 133 113.5) (end 137 117.5) (width 0.2) (layer "F.Cu") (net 47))
 (segment (start 121 111) (end 121.5 110.5) (width 0.2) (layer "F.Cu") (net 3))
 (segment (start 119.15 111) (end 121 111) (width 0.2) (layer "F.Cu") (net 3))
 (segment (start 114.85 111) (end 113 111) (width 0.2) (layer "F.Cu") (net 4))
 (segment (start 113 111) (end 112.5 110.5) (width 0.2) (layer "F.Cu") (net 4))
 (segment (start 113.5 111.5) (end 112.5 112.5) (width 0.2) (layer "F.Cu") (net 6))
 (segment (start 114.85 111.5) (end 113.5 111.5) (width 0.2) (layer "F.Cu") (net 6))
 (segment (start 119.15 112.5) (end 121.5 112.5) (width 0.2) (layer "F.Cu") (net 5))
 (segment (start 147.575 107.365) (end 149.635 107.365) (width 0.2) (layer "F.Cu") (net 2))
 (segment (start 149.635 107.365) (end 150 107) (width 0.2) (layer "F.Cu") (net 2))
 (segment (start 119.8 113) (end 120.8 114) (width 0.2) (layer "F.Cu") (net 45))
 (segment (start 119.15 113) (end 119.8 113) (width 0.2) (layer "F.Cu") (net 45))
 (segment (start 119.15 113) (end 119 113) (width 0.2) (layer "F.Cu") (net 45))
 (segment (start 147.67 106) (end 147.575 106.095) (width 0.2) (layer "F.Cu") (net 51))
 (segment (start 150 106) (end 147.67 106) (width 0.2) (layer "F.Cu") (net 51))
 (segment (start 149.635 108.635) (end 150 109) (width 0.2) (layer "F.Cu") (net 50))
 (segment (start 147.575 108.635) (end 149.635 108.635) (width 0.2) (layer "F.Cu") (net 50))
 (segment (start 150 109) (end 151 109) (width 0.2) (layer "F.Cu") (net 50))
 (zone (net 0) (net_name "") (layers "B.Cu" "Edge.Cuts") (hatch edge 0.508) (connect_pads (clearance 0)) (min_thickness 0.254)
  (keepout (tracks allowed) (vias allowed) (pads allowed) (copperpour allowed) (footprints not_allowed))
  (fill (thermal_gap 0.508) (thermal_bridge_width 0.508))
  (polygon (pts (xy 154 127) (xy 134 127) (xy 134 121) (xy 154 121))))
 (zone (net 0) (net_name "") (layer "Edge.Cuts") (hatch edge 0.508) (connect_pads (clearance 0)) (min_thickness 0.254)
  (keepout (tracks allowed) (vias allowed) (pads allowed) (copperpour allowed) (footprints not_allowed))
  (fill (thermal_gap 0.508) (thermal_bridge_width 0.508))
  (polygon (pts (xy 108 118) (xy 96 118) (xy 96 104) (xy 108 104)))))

